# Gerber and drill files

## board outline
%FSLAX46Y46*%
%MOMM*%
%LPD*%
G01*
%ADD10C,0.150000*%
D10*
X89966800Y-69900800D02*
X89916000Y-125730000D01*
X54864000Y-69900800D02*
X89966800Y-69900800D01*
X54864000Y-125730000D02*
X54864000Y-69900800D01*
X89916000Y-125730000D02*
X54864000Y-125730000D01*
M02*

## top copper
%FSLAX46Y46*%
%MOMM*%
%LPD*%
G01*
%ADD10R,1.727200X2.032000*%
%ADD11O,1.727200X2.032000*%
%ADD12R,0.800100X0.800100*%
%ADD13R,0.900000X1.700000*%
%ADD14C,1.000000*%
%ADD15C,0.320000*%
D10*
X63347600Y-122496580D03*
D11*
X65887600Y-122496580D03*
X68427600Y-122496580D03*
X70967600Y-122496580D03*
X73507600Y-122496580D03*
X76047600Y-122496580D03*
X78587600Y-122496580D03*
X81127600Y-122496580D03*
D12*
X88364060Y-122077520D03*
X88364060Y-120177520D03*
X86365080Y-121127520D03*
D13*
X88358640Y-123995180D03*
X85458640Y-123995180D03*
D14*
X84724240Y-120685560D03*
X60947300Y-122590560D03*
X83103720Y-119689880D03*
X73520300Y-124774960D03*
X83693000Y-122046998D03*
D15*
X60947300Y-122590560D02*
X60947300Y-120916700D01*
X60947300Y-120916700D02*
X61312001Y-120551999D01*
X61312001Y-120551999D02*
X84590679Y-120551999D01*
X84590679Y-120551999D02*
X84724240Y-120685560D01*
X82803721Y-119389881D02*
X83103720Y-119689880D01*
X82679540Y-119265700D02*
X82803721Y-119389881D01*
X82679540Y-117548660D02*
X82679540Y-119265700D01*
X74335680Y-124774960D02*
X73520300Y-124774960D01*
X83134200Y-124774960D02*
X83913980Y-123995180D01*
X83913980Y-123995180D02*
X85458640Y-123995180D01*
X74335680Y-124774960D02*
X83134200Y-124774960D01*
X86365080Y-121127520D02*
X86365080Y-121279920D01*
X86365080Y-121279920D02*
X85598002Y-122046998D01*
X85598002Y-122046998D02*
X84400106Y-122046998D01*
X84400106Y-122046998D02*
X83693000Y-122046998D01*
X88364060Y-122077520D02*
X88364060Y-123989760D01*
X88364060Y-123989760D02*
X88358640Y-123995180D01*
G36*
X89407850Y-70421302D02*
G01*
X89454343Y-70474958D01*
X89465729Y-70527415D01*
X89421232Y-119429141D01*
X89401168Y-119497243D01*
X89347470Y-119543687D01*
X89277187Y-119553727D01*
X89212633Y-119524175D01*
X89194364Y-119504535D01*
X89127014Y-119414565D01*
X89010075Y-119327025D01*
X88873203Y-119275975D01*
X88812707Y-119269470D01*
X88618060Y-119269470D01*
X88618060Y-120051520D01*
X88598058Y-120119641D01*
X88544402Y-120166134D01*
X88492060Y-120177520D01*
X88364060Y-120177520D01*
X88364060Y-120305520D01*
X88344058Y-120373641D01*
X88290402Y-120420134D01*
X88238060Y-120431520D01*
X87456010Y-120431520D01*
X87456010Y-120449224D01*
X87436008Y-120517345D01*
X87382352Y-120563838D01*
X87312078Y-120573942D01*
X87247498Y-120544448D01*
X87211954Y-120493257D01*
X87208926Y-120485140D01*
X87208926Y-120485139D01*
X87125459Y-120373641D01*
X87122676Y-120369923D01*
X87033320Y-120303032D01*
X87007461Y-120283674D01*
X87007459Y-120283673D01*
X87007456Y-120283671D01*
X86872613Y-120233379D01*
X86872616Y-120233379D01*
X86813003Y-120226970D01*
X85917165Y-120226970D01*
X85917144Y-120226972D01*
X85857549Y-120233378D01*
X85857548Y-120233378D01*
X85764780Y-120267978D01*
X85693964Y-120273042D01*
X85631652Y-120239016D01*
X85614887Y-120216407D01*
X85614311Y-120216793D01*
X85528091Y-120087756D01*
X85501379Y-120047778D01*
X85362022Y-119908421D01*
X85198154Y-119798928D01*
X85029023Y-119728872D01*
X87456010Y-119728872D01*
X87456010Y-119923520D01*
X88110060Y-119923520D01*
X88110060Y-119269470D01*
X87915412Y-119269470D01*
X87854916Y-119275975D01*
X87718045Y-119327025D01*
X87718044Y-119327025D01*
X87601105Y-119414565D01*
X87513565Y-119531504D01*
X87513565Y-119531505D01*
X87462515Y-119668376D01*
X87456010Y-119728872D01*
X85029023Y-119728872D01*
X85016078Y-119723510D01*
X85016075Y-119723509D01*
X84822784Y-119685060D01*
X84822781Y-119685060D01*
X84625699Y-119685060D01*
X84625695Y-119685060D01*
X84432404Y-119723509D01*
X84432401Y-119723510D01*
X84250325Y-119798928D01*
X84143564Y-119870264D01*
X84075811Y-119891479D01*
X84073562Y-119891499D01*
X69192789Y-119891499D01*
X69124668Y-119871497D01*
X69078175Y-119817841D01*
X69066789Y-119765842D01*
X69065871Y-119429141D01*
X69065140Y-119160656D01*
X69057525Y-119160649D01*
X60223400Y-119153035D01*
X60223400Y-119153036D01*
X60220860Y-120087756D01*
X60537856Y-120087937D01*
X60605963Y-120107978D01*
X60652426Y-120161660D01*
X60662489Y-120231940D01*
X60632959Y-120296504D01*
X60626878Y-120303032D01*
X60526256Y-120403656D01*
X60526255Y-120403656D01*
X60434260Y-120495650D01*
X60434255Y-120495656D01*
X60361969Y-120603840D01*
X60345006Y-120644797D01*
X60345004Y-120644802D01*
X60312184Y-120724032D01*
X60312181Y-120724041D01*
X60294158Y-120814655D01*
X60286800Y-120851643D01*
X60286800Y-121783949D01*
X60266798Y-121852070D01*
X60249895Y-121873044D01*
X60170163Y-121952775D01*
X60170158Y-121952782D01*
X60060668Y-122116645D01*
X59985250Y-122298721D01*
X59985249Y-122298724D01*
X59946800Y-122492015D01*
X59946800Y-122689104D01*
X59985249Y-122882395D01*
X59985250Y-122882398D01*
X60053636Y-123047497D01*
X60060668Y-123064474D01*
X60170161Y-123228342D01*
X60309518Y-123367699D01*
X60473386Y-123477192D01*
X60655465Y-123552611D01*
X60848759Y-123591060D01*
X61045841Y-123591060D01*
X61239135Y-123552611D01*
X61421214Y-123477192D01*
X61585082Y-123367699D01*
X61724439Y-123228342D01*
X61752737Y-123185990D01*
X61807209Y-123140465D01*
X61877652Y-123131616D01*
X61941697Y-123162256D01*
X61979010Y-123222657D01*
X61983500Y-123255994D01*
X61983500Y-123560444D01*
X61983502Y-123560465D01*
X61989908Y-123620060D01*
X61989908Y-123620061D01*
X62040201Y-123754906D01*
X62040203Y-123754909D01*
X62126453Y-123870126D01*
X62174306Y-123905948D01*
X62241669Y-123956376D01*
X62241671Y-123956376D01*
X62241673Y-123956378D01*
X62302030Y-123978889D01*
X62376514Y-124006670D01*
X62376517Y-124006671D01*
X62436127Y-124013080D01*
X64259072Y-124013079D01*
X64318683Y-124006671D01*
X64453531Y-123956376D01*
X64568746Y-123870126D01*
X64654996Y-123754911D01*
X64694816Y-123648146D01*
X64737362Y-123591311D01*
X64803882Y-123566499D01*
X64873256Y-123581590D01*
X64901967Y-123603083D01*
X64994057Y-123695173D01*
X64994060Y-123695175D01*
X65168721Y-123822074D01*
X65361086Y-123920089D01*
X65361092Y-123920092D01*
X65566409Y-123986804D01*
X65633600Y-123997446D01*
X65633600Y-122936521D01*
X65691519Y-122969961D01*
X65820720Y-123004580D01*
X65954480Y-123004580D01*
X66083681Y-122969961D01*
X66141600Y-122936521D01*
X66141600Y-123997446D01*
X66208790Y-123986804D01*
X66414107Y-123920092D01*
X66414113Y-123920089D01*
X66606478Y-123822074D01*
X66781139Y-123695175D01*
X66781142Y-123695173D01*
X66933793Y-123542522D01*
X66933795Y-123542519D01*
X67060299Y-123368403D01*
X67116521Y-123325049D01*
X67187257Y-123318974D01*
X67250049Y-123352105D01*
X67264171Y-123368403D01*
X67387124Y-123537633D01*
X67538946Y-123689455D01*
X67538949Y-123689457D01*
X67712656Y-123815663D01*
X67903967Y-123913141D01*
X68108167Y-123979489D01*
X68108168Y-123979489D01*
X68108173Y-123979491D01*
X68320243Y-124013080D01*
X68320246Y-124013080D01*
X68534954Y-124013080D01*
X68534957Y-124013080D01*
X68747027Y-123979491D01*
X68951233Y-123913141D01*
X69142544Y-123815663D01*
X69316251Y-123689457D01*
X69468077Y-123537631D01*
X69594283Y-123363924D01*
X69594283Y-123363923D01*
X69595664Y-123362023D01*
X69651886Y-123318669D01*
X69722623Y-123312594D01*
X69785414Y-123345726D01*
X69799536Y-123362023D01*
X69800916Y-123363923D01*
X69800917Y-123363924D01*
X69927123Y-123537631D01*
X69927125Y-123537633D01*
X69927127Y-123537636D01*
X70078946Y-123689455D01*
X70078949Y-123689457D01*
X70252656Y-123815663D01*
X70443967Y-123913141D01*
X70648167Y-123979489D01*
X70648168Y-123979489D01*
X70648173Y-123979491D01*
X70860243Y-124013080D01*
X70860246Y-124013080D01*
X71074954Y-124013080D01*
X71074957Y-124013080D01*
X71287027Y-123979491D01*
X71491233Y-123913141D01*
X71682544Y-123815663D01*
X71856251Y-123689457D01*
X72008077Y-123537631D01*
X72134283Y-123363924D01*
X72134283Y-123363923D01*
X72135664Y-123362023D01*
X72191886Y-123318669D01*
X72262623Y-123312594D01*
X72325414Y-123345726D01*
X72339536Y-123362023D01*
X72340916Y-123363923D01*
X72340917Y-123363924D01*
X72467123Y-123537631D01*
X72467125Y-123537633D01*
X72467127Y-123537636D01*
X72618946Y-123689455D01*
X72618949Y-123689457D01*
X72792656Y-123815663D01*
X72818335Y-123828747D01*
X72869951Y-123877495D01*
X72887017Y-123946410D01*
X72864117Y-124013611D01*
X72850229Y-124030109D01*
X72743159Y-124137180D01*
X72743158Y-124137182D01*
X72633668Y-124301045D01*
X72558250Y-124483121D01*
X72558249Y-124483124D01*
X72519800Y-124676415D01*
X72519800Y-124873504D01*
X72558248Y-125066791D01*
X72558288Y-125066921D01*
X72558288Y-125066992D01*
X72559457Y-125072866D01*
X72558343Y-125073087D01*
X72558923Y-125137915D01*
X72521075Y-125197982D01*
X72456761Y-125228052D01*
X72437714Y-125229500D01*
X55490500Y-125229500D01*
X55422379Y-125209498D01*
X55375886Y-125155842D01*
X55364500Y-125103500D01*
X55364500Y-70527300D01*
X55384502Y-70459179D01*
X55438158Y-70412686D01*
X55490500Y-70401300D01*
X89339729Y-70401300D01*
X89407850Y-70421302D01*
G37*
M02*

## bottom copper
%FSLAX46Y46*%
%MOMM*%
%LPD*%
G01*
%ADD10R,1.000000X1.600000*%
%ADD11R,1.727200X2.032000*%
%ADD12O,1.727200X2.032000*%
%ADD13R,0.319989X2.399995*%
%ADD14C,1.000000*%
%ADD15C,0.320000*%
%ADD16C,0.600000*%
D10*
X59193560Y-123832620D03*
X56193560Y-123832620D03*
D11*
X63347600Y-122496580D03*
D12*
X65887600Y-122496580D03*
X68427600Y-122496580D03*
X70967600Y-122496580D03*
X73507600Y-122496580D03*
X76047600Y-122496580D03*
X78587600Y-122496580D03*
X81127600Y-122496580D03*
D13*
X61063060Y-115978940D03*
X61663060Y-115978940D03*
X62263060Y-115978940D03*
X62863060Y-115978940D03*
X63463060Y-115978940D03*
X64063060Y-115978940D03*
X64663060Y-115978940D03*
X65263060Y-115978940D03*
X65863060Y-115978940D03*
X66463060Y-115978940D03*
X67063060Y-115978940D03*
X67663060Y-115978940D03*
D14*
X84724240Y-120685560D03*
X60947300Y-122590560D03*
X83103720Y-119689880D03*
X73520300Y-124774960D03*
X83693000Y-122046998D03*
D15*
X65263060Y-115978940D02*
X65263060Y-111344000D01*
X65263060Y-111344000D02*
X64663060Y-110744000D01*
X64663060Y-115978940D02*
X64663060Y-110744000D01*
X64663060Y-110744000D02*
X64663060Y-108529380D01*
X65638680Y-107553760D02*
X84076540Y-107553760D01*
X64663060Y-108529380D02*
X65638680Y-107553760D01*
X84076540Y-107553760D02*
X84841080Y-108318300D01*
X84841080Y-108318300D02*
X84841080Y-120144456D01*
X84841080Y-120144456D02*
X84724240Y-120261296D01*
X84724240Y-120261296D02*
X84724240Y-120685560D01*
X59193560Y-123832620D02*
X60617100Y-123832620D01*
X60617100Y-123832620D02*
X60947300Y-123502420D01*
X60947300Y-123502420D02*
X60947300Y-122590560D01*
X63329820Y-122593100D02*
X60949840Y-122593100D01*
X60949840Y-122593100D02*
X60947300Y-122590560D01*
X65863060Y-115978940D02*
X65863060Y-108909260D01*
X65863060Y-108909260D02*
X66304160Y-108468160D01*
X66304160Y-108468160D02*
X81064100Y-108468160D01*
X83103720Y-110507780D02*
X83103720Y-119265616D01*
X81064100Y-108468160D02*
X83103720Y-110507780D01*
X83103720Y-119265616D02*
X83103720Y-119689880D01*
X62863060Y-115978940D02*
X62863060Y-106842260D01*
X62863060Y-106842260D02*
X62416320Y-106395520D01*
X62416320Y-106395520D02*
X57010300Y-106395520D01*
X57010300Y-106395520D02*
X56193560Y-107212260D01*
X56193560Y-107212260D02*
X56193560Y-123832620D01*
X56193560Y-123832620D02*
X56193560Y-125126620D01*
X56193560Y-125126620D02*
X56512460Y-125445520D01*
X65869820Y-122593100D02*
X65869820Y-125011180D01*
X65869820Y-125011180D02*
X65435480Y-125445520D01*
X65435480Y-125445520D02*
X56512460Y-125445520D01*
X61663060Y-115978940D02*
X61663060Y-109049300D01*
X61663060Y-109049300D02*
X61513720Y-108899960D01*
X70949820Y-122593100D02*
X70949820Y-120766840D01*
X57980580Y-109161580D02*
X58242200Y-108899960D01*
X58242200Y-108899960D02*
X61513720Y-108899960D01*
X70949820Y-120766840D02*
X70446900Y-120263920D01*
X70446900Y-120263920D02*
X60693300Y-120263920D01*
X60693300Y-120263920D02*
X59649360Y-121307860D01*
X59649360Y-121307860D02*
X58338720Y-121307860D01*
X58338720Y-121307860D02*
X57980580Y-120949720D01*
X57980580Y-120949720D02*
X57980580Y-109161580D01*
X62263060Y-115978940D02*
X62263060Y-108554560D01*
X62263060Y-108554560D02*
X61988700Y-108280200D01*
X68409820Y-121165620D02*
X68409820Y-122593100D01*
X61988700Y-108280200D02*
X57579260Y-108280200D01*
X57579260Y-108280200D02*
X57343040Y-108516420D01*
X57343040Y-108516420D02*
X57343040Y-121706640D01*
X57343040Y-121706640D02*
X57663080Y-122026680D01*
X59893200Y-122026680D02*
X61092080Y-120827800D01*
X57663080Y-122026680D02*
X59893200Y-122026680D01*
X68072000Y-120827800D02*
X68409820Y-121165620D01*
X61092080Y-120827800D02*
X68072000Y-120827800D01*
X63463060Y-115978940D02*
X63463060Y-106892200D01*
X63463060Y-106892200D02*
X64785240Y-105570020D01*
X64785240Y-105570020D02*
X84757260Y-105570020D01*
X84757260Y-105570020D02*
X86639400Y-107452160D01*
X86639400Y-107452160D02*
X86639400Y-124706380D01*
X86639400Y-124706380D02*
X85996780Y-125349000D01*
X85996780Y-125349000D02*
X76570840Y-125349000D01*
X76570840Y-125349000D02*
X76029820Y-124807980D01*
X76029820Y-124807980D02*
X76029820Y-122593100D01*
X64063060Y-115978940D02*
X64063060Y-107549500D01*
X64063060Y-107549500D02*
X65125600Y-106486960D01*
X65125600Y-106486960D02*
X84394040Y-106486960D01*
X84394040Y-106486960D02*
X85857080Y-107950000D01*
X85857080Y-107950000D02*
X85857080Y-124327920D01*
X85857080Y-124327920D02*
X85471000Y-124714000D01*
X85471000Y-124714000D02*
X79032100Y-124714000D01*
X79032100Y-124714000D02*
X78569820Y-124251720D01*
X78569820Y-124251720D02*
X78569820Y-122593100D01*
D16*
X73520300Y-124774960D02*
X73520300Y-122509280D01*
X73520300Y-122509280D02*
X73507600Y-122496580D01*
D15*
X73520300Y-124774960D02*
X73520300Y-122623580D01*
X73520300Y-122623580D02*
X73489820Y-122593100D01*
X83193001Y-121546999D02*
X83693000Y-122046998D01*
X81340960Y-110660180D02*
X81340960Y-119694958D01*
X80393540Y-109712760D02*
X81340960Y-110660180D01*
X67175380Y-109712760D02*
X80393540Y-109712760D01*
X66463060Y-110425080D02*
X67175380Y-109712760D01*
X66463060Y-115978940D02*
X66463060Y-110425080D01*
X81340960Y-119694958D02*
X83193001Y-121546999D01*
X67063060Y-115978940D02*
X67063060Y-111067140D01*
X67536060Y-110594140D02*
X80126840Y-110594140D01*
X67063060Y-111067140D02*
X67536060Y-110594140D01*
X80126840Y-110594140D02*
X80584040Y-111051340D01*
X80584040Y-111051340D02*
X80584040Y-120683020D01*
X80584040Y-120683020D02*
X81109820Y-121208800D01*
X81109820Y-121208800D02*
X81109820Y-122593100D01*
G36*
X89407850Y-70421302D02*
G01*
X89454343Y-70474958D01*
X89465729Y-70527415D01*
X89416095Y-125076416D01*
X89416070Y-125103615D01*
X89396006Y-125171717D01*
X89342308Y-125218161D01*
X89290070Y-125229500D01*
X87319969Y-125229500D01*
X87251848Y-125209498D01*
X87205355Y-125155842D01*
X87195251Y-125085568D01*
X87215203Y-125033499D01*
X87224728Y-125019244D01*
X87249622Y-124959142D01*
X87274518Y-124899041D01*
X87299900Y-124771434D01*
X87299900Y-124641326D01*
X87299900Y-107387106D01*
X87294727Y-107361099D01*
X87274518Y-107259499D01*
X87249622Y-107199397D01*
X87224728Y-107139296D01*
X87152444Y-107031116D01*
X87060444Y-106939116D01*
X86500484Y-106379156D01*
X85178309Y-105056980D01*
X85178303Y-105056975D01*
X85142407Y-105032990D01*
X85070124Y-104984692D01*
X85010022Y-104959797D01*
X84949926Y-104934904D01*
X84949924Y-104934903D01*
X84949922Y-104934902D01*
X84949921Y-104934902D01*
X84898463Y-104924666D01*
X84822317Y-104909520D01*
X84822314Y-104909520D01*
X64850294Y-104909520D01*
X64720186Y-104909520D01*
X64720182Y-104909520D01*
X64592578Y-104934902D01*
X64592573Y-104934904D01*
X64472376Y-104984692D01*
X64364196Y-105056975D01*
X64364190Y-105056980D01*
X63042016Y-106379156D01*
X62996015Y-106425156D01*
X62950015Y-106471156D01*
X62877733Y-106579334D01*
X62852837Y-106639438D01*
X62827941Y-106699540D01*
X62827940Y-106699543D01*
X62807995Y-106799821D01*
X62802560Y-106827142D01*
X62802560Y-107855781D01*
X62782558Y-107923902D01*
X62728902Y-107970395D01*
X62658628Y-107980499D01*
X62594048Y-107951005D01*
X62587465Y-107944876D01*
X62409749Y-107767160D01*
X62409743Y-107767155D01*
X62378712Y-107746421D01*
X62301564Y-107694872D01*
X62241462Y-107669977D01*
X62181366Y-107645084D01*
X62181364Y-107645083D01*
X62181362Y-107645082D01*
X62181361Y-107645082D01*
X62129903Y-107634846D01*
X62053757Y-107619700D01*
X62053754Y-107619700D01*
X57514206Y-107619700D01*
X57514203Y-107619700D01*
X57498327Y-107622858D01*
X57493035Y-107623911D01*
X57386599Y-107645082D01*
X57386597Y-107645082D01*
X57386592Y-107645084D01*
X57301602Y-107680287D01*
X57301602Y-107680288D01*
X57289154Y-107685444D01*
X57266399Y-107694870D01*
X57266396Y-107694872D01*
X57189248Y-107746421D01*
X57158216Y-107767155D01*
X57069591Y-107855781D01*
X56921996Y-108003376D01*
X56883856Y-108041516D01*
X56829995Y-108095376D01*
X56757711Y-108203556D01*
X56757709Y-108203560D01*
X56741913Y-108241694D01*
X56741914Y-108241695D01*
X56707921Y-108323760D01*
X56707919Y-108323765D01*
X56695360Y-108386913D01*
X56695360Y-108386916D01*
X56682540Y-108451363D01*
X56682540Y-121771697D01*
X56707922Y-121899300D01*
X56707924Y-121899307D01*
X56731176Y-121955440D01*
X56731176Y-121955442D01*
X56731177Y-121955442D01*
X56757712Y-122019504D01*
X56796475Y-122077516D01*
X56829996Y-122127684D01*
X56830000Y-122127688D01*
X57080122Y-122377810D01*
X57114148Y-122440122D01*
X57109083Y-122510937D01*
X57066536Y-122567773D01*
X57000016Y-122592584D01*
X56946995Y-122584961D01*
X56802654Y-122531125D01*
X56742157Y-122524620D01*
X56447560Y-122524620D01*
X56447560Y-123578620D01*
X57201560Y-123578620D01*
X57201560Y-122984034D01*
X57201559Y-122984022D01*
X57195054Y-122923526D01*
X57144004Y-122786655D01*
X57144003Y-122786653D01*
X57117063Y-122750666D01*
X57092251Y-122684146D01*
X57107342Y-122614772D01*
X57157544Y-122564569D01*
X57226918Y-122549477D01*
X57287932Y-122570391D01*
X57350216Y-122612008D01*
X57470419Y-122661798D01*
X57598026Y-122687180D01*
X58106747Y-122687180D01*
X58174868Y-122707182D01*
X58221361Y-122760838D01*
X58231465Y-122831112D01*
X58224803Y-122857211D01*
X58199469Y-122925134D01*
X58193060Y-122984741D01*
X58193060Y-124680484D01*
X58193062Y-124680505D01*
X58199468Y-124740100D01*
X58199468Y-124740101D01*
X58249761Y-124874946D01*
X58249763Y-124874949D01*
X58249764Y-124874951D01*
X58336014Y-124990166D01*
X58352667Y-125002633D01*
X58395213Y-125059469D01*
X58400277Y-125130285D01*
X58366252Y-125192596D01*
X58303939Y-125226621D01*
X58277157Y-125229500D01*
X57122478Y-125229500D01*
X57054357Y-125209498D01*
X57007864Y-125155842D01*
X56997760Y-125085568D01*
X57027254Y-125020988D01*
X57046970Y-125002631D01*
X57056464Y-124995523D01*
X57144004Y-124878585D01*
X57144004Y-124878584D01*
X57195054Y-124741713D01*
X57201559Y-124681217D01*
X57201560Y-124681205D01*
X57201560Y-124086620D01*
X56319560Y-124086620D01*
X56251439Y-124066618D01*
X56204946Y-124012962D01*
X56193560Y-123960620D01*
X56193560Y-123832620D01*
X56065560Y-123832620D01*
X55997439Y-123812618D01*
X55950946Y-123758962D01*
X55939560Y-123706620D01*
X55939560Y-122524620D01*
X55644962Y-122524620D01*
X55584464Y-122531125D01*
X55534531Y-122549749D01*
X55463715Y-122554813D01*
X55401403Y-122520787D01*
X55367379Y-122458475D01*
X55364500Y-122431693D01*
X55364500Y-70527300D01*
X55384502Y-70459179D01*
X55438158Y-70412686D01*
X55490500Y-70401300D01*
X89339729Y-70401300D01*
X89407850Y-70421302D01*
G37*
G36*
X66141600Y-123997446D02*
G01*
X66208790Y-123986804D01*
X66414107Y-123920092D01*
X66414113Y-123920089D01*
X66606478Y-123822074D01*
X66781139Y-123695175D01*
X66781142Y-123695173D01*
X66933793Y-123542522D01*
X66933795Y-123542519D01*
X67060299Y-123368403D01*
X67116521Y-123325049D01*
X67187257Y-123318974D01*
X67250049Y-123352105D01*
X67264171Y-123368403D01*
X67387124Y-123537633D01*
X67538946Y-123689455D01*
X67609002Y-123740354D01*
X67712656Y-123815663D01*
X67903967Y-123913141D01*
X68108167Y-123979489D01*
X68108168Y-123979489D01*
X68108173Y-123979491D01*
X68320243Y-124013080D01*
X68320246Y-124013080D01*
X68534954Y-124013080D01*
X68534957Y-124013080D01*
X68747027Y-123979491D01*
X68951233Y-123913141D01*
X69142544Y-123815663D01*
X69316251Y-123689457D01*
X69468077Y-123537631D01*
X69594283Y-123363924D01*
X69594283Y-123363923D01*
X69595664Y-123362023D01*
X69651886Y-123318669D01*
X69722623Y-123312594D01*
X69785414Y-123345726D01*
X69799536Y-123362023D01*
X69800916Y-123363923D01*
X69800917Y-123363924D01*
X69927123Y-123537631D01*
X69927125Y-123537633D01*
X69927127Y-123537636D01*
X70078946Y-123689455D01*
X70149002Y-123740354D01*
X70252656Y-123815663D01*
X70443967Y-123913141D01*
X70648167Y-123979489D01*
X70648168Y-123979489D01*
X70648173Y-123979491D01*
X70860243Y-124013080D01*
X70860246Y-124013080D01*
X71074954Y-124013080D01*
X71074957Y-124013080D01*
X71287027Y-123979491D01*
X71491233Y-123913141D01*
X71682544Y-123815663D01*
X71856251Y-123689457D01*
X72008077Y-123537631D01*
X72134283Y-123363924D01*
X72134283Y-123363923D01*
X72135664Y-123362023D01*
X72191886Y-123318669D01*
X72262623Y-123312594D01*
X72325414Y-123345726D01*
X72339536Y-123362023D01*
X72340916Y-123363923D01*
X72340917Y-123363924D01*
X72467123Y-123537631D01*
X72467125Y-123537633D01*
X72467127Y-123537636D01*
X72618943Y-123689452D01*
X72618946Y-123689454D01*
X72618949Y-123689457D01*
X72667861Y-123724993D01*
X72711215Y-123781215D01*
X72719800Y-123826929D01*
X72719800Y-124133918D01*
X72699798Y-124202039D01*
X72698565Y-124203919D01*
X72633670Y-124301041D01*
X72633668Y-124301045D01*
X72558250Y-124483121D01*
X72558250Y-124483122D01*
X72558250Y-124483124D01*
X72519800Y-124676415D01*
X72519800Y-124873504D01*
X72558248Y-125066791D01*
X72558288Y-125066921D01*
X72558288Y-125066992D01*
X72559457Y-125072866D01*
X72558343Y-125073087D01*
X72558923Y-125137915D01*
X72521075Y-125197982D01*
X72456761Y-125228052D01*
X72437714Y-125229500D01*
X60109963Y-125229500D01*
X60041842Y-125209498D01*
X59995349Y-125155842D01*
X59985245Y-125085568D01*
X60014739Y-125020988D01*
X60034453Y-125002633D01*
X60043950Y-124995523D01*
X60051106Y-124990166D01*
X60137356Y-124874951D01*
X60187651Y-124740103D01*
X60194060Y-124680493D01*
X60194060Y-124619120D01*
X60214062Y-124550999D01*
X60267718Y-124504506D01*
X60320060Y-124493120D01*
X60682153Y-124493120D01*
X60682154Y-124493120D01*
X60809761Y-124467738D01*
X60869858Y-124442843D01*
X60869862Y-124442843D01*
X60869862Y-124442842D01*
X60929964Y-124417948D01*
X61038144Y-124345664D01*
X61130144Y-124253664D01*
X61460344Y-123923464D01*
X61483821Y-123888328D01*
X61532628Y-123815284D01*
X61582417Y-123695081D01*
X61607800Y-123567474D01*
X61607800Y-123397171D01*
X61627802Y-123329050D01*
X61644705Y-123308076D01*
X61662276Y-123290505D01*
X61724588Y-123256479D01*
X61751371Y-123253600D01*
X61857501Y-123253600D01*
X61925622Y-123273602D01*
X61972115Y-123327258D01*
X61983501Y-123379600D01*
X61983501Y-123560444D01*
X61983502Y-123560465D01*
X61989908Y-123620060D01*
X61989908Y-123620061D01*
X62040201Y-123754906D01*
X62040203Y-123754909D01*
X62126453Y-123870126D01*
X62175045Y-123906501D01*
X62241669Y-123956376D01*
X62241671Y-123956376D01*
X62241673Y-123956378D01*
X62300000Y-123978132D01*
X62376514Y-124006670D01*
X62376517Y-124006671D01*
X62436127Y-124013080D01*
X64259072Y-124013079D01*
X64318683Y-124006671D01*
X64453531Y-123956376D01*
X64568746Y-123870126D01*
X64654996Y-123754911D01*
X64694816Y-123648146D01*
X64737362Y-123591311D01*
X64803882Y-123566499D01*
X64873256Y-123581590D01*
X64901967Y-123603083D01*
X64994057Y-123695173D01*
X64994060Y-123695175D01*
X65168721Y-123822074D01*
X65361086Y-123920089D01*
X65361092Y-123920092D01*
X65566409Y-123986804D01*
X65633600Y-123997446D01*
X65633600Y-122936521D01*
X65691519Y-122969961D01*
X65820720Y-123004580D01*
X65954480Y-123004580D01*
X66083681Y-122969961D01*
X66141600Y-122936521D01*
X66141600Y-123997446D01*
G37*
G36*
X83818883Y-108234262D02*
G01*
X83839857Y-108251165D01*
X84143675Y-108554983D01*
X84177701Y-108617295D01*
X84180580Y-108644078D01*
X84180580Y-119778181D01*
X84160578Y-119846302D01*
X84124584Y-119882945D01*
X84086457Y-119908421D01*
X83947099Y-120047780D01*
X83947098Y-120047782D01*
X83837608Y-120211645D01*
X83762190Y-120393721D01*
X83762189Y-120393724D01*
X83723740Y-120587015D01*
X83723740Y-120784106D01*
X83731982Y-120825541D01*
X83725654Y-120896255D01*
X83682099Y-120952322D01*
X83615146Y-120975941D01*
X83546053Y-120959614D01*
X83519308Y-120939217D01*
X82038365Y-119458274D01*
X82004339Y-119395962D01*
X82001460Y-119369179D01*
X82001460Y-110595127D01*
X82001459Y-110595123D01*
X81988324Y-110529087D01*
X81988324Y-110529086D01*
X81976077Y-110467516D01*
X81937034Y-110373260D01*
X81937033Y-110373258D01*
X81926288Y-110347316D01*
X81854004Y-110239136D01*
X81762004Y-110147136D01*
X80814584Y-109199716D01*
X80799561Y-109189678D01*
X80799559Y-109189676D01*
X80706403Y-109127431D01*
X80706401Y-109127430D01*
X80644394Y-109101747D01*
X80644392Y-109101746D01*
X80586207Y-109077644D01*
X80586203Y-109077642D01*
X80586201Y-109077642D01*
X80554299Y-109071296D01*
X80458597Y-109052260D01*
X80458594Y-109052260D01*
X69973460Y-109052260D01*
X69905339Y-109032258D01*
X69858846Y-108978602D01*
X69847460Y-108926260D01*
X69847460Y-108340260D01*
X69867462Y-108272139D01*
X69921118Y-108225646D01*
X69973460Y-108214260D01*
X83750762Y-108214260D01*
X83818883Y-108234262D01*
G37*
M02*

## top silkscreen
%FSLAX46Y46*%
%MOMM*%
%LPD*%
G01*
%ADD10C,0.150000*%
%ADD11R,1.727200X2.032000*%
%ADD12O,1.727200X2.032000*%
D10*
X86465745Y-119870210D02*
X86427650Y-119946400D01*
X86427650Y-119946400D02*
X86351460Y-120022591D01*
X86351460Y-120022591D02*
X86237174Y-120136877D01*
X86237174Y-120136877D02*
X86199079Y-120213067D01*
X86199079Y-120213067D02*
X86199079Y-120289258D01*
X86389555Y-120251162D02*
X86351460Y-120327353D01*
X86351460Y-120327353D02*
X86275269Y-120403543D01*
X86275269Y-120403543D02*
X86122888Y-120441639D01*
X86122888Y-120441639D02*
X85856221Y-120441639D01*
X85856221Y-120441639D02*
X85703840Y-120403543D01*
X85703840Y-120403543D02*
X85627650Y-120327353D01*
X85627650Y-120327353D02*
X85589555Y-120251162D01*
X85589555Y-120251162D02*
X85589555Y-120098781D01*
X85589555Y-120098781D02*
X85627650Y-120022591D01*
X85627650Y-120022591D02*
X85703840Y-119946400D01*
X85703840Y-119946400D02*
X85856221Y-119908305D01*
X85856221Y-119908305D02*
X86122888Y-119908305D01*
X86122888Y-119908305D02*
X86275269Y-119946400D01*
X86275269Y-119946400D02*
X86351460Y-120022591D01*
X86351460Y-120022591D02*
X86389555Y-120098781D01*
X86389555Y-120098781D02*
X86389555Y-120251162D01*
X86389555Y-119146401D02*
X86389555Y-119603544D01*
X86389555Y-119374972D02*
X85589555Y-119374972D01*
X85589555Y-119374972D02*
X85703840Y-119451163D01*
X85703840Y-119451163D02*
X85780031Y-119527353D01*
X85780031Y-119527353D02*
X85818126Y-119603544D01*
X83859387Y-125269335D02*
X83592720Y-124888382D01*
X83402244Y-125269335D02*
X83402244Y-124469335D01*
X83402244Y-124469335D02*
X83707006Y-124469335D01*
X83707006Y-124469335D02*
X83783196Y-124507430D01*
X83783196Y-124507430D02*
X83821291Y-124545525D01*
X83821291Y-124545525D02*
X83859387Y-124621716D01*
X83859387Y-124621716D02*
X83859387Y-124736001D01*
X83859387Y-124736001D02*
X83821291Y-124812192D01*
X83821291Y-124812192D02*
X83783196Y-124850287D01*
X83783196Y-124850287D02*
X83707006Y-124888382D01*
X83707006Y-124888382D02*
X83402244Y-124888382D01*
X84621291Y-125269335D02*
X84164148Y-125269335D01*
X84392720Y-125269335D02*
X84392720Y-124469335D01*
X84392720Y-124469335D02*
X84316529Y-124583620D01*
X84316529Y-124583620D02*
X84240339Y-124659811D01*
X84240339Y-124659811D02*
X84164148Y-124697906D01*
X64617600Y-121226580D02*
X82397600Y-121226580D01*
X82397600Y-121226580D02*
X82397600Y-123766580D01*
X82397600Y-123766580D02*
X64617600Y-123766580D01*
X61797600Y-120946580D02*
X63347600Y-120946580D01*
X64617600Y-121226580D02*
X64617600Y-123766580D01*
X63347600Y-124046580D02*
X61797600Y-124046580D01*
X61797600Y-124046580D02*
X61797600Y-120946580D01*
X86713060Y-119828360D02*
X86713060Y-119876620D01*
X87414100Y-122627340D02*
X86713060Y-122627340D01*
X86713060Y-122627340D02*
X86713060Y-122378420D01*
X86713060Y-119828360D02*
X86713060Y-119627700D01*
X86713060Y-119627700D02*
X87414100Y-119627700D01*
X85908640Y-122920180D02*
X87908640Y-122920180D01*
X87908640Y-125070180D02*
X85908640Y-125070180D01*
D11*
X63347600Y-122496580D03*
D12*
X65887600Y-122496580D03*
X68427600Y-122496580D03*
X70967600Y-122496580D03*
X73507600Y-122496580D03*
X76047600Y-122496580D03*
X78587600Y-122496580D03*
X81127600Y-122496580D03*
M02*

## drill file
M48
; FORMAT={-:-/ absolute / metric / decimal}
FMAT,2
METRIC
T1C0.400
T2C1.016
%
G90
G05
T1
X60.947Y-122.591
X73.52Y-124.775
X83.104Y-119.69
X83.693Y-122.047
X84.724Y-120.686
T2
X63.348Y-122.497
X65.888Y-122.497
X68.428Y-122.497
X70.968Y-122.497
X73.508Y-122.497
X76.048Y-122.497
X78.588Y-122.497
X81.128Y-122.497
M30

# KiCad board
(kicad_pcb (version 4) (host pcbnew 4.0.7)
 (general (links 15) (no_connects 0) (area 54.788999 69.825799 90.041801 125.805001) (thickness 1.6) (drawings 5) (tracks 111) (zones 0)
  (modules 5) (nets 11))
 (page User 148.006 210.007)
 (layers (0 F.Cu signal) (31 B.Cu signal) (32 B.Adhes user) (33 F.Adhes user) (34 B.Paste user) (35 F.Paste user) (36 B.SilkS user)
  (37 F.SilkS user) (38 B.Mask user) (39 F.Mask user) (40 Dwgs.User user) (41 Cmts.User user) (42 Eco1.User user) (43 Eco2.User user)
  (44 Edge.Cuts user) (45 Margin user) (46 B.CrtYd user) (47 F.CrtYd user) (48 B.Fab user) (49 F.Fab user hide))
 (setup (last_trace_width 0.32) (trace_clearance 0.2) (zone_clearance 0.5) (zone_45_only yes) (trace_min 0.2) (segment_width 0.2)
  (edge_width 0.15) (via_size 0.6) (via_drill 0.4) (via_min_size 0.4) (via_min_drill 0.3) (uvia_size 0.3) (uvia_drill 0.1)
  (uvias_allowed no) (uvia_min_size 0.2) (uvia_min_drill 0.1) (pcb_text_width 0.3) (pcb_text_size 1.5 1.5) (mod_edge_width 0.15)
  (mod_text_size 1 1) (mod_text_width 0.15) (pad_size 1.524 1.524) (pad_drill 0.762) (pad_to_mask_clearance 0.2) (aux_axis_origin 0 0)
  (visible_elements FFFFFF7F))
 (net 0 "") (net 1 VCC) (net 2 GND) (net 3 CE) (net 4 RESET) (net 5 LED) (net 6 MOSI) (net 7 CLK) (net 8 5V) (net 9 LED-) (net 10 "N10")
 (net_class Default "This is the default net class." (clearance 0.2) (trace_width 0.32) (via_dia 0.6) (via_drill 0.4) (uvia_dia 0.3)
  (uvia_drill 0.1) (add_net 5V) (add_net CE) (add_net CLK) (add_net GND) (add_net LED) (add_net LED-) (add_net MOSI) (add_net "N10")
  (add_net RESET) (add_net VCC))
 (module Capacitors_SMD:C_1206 (layer B.Cu) (at 57.69356 123.83262 180)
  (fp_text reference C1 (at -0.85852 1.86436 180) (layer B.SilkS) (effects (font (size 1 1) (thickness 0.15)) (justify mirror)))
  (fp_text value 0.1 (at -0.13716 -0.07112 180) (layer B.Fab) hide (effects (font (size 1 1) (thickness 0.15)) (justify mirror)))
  (pad 1 smd rect (at -1.5 0 180) (size 1 1.6) (layers B.Cu B.Paste B.Mask) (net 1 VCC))
  (pad 2 smd rect (at 1.5 0 180) (size 1 1.6) (layers B.Cu B.Paste B.Mask) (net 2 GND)))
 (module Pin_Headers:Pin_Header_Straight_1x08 (layer F.Cu) (at 63.3476 122.49658 90)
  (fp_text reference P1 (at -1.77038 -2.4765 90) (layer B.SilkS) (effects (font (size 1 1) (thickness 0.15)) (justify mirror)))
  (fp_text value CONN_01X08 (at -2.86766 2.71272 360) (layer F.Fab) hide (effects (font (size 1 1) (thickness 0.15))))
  (fp_line (start 1.27 1.27) (end 1.27 19.05) (layer F.SilkS) (width 0.15))
  (fp_line (start 1.27 19.05) (end -1.27 19.05) (layer F.SilkS) (width 0.15))
  (fp_line (start -1.27 19.05) (end -1.27 1.27) (layer F.SilkS) (width 0.15))
  (fp_line (start 1.55 -1.55) (end 1.55 0) (layer F.SilkS) (width 0.15))
  (fp_line (start 1.27 1.27) (end -1.27 1.27) (layer F.SilkS) (width 0.15))
  (fp_line (start -1.55 0) (end -1.55 -1.55) (layer F.SilkS) (width 0.15))
  (fp_line (start -1.55 -1.55) (end 1.55 -1.55) (layer F.SilkS) (width 0.15))
  (pad 1 thru_hole rect (at 0 0 90) (size 2.032 1.7272) (drill 1.016) (layers *.Cu *.Mask F.SilkS) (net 1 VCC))
  (pad 2 thru_hole oval (at 0 2.54 90) (size 2.032 1.7272) (drill 1.016) (layers *.Cu *.Mask F.SilkS) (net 2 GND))
  (pad 3 thru_hole oval (at 0 5.08 90) (size 2.032 1.7272) (drill 1.016) (layers *.Cu *.Mask F.SilkS) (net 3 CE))
  (pad 4 thru_hole oval (at 0 7.62 90) (size 2.032 1.7272) (drill 1.016) (layers *.Cu *.Mask F.SilkS) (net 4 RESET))
  (pad 5 thru_hole oval (at 0 10.16 90) (size 2.032 1.7272) (drill 1.016) (layers *.Cu *.Mask F.SilkS) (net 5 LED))
  (pad 6 thru_hole oval (at 0 12.7 90) (size 2.032 1.7272) (drill 1.016) (layers *.Cu *.Mask F.SilkS) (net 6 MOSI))
  (pad 7 thru_hole oval (at 0 15.24 90) (size 2.032 1.7272) (drill 1.016) (layers *.Cu *.Mask F.SilkS) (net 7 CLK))
  (pad 8 thru_hole oval (at 0 17.78 90) (size 2.032 1.7272) (drill 1.016) (layers *.Cu *.Mask F.SilkS) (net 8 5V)))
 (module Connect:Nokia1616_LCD (layer B.Cu) (at 68.14454 114.77752)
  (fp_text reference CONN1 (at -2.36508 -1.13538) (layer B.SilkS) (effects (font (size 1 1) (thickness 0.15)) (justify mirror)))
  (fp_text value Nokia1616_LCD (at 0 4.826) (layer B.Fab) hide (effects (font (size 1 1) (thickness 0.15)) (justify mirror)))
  (pad 1 smd rect (at -7.08148 1.20142) (size 0.319989 2.399995) (layers B.Cu B.Paste B.Mask))
  (pad 2 smd rect (at -6.48148 1.20142) (size 0.319989 2.399995) (layers B.Cu B.Paste B.Mask) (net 4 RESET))
  (pad 3 smd rect (at -5.88148 1.20142) (size 0.319989 2.399995) (layers B.Cu B.Paste B.Mask) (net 3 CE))
  (pad 4 smd rect (at -5.28148 1.20142) (size 0.319989 2.399995) (layers B.Cu B.Paste B.Mask) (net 2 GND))
  (pad 5 smd rect (at -4.68148 1.20142) (size 0.319989 2.399995) (layers B.Cu B.Paste B.Mask) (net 6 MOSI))
  (pad 6 smd rect (at -4.08148 1.20142) (size 0.319989 2.399995) (layers B.Cu B.Paste B.Mask) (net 7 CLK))
  (pad 7 smd rect (at -3.48148 1.20142) (size 0.319989 2.399995) (layers B.Cu B.Paste B.Mask) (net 1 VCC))
  (pad 8 smd rect (at -2.88148 1.20142) (size 0.319989 2.399995) (layers B.Cu B.Paste B.Mask) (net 1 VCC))
  (pad 9 smd rect (at -2.28148 1.20142) (size 0.319989 2.399995) (layers B.Cu B.Paste B.Mask) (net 2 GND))
  (pad 10 smd rect (at -1.68148 1.20142) (size 0.319989 2.399995) (layers B.Cu B.Paste B.Mask) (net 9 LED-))
  (pad 11 smd rect (at -1.08148 1.20142) (size 0.319989 2.399995) (layers B.Cu B.Paste B.Mask) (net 8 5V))
  (pad 12 smd rect (at -0.48148 1.20142) (size 0.319989 2.399995) (layers B.Cu B.Paste B.Mask)))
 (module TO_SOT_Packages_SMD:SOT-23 (layer F.Cu) (at 87.3633 121.12752 90)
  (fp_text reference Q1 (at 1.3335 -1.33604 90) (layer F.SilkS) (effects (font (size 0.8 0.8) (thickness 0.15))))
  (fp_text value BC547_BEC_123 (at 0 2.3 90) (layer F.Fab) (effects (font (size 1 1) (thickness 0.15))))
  (fp_line (start 1.29916 -0.65024) (end 1.2509 -0.65024) (layer F.SilkS) (width 0.15))
  (fp_line (start -1.49982 0.0508) (end -1.49982 -0.65024) (layer F.SilkS) (width 0.15))
  (fp_line (start -1.49982 -0.65024) (end -1.2509 -0.65024) (layer F.SilkS) (width 0.15))
  (fp_line (start 1.29916 -0.65024) (end 1.49982 -0.65024) (layer F.SilkS) (width 0.15))
  (fp_line (start 1.49982 -0.65024) (end 1.49982 0.0508) (layer F.SilkS) (width 0.15))
  (pad 1 smd rect (at -0.95 1.00076 90) (size 0.8001 0.8001) (layers F.Cu F.Paste F.Mask) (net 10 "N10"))
  (pad 2 smd rect (at 0.95 1.00076 90) (size 0.8001 0.8001) (layers F.Cu F.Paste F.Mask) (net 2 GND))
  (pad 3 smd rect (at 0 -0.99822 90) (size 0.8001 0.8001) (layers F.Cu F.Paste F.Mask) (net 9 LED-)))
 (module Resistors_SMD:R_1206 (layer F.Cu) (at 86.90864 123.99518 180)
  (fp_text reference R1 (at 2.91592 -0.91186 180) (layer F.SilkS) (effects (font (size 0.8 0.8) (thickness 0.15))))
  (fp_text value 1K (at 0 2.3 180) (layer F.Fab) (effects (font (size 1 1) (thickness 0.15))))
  (fp_line (start 1 1.075) (end -1 1.075) (layer F.SilkS) (width 0.15))
  (fp_line (start -1 -1.075) (end 1 -1.075) (layer F.SilkS) (width 0.15))
  (pad 1 smd rect (at -1.45 0 180) (size 0.9 1.7) (layers F.Cu F.Paste F.Mask) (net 10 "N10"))
  (pad 2 smd rect (at 1.45 0 180) (size 0.9 1.7) (layers F.Cu F.Paste F.Mask) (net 5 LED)))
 (gr_line (start 89.9668 69.9008) (end 89.916 125.73) (layer Edge.Cuts) (width 0.15))
 (gr_line (start 54.864 69.9008) (end 89.9668 69.9008) (layer Edge.Cuts) (width 0.15))
 (gr_line (start 54.864 125.73) (end 54.864 69.9008) (layer Edge.Cuts) (width 0.15))
 (gr_line (start 89.916 125.73) (end 54.864 125.73) (layer Edge.Cuts) (width 0.15))
 (segment (start 60.9473 122.59056) (end 60.9473 120.9167) (width 0.32) (layer F.Cu) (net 1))
 (segment (start 60.9473 120.9167) (end 61.312001 120.551999) (width 0.32) (layer F.Cu) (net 1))
 (segment (start 61.312001 120.551999) (end 84.590679 120.551999) (width 0.32) (layer F.Cu) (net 1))
 (segment (start 84.590679 120.551999) (end 84.72424 120.68556) (width 0.32) (layer F.Cu) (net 1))
 (segment (start 65.26306 115.97894) (end 65.26306 111.344) (width 0.32) (layer B.Cu) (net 1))
 (segment (start 65.26306 111.344) (end 64.66306 110.744) (width 0.32) (layer B.Cu) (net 1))
 (segment (start 64.66306 115.97894) (end 64.66306 110.744) (width 0.32) (layer B.Cu) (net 1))
 (segment (start 64.66306 110.744) (end 64.66306 108.52938) (width 0.32) (layer B.Cu) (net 1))
 (segment (start 65.63868 107.55376) (end 84.07654 107.55376) (width 0.32) (layer B.Cu) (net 1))
 (segment (start 64.66306 108.52938) (end 65.63868 107.55376) (width 0.32) (layer B.Cu) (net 1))
 (segment (start 84.07654 107.55376) (end 84.84108 108.3183) (width 0.32) (layer B.Cu) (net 1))
 (segment (start 84.84108 108.3183) (end 84.84108 120.144456) (width 0.32) (layer B.Cu) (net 1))
 (segment (start 84.84108 120.144456) (end 84.72424 120.261296) (width 0.32) (layer B.Cu) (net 1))
 (segment (start 84.72424 120.261296) (end 84.72424 120.68556) (width 0.32) (layer B.Cu) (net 1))
 (segment (start 59.19356 123.83262) (end 60.6171 123.83262) (width 0.32) (layer B.Cu) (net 1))
 (segment (start 60.6171 123.83262) (end 60.9473 123.50242) (width 0.32) (layer B.Cu) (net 1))
 (segment (start 60.9473 123.50242) (end 60.9473 122.59056) (width 0.32) (layer B.Cu) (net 1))
 (via (at 84.72424 120.68556) (size 1) (drill 0.4) (layers F.Cu B.Cu) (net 1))
 (segment (start 63.32982 122.5931) (end 60.94984 122.5931) (width 0.32) (layer B.Cu) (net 1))
 (segment (start 60.94984 122.5931) (end 60.9473 122.59056) (width 0.32) (layer B.Cu) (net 1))
 (via (at 60.9473 122.59056) (size 1) (drill 0.4) (layers F.Cu B.Cu) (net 1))
 (segment (start 65.86306 115.97894) (end 65.86306 108.90926) (width 0.32) (layer B.Cu) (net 2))
 (segment (start 65.86306 108.90926) (end 66.30416 108.46816) (width 0.32) (layer B.Cu) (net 2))
 (segment (start 66.30416 108.46816) (end 81.0641 108.46816) (width 0.32) (layer B.Cu) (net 2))
 (segment (start 83.10372 110.50778) (end 83.10372 119.265616) (width 0.32) (layer B.Cu) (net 2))
 (segment (start 81.0641 108.46816) (end 83.10372 110.50778) (width 0.32) (layer B.Cu) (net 2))
 (segment (start 83.10372 119.265616) (end 83.10372 119.68988) (width 0.32) (layer B.Cu) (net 2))
 (segment (start 62.86306 115.97894) (end 62.86306 106.84226) (width 0.32) (layer B.Cu) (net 2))
 (segment (start 62.86306 106.84226) (end 62.41632 106.39552) (width 0.32) (layer B.Cu) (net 2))
 (segment (start 62.41632 106.39552) (end 57.0103 106.39552) (width 0.32) (layer B.Cu) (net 2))
 (segment (start 57.0103 106.39552) (end 56.19356 107.21226) (width 0.32) (layer B.Cu) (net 2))
 (segment (start 56.19356 107.21226) (end 56.19356 123.83262) (width 0.32) (layer B.Cu) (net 2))
 (segment (start 56.19356 123.83262) (end 56.19356 125.12662) (width 0.32) (layer B.Cu) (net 2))
 (segment (start 56.19356 125.12662) (end 56.51246 125.44552) (width 0.32) (layer B.Cu) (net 2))
 (segment (start 65.86982 122.5931) (end 65.86982 125.01118) (width 0.32) (layer B.Cu) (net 2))
 (segment (start 65.86982 125.01118) (end 65.43548 125.44552) (width 0.32) (layer B.Cu) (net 2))
 (segment (start 65.43548 125.44552) (end 56.51246 125.44552) (width 0.32) (layer B.Cu) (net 2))
 (segment (start 82.803721 119.389881) (end 83.10372 119.68988) (width 0.32) (layer F.Cu) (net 2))
 (segment (start 82.67954 119.2657) (end 82.803721 119.389881) (width 0.32) (layer F.Cu) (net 2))
 (segment (start 82.67954 117.54866) (end 82.67954 119.2657) (width 0.32) (layer F.Cu) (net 2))
 (via (at 83.10372 119.68988) (size 1) (drill 0.4) (layers F.Cu B.Cu) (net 2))
 (segment (start 61.66306 115.97894) (end 61.66306 109.0493) (width 0.32) (layer B.Cu) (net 4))
 (segment (start 61.66306 109.0493) (end 61.51372 108.89996) (width 0.32) (layer B.Cu) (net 4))
 (segment (start 70.94982 122.5931) (end 70.94982 120.76684) (width 0.32) (layer B.Cu) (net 4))
 (segment (start 57.98058 109.16158) (end 58.2422 108.89996) (width 0.32) (layer B.Cu) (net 4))
 (segment (start 58.2422 108.89996) (end 61.51372 108.89996) (width 0.32) (layer B.Cu) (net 4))
 (segment (start 70.94982 120.76684) (end 70.4469 120.26392) (width 0.32) (layer B.Cu) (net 4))
 (segment (start 70.4469 120.26392) (end 60.6933 120.26392) (width 0.32) (layer B.Cu) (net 4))
 (segment (start 60.6933 120.26392) (end 59.64936 121.30786) (width 0.32) (layer B.Cu) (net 4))
 (segment (start 59.64936 121.30786) (end 58.33872 121.30786) (width 0.32) (layer B.Cu) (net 4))
 (segment (start 58.33872 121.30786) (end 57.98058 120.94972) (width 0.32) (layer B.Cu) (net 4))
 (segment (start 57.98058 120.94972) (end 57.98058 109.16158) (width 0.32) (layer B.Cu) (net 4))
 (segment (start 62.26306 115.97894) (end 62.26306 108.55456) (width 0.32) (layer B.Cu) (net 3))
 (segment (start 62.26306 108.55456) (end 61.9887 108.2802) (width 0.32) (layer B.Cu) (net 3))
 (segment (start 68.40982 121.16562) (end 68.40982 122.5931) (width 0.32) (layer B.Cu) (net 3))
 (segment (start 61.9887 108.2802) (end 57.57926 108.2802) (width 0.32) (layer B.Cu) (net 3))
 (segment (start 57.57926 108.2802) (end 57.34304 108.51642) (width 0.32) (layer B.Cu) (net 3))
 (segment (start 57.34304 108.51642) (end 57.34304 121.70664) (width 0.32) (layer B.Cu) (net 3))
 (segment (start 57.34304 121.70664) (end 57.66308 122.02668) (width 0.32) (layer B.Cu) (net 3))
 (segment (start 59.8932 122.02668) (end 61.09208 120.8278) (width 0.32) (layer B.Cu) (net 3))
 (segment (start 57.66308 122.02668) (end 59.8932 122.02668) (width 0.32) (layer B.Cu) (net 3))
 (segment (start 68.072 120.8278) (end 68.40982 121.16562) (width 0.32) (layer B.Cu) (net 3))
 (segment (start 61.09208 120.8278) (end 68.072 120.8278) (width 0.32) (layer B.Cu) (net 3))
 (segment (start 63.46306 115.97894) (end 63.46306 106.8922) (width 0.32) (layer B.Cu) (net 6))
 (segment (start 63.46306 106.8922) (end 64.78524 105.57002) (width 0.32) (layer B.Cu) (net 6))
 (segment (start 64.78524 105.57002) (end 84.75726 105.57002) (width 0.32) (layer B.Cu) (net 6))
 (segment (start 84.75726 105.57002) (end 86.6394 107.45216) (width 0.32) (layer B.Cu) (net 6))
 (segment (start 86.6394 107.45216) (end 86.6394 124.70638) (width 0.32) (layer B.Cu) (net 6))
 (segment (start 86.6394 124.70638) (end 85.99678 125.349) (width 0.32) (layer B.Cu) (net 6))
 (segment (start 85.99678 125.349) (end 76.57084 125.349) (width 0.32) (layer B.Cu) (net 6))
 (segment (start 76.57084 125.349) (end 76.02982 124.80798) (width 0.32) (layer B.Cu) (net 6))
 (segment (start 76.02982 124.80798) (end 76.02982 122.5931) (width 0.32) (layer B.Cu) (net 6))
 (segment (start 64.06306 115.97894) (end 64.06306 107.5495) (width 0.32) (layer B.Cu) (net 7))
 (segment (start 64.06306 107.5495) (end 65.1256 106.48696) (width 0.32) (layer B.Cu) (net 7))
 (segment (start 65.1256 106.48696) (end 84.39404 106.48696) (width 0.32) (layer B.Cu) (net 7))
 (segment (start 84.39404 106.48696) (end 85.85708 107.95) (width 0.32) (layer B.Cu) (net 7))
 (segment (start 85.85708 107.95) (end 85.85708 124.32792) (width 0.32) (layer B.Cu) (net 7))
 (segment (start 85.85708 124.32792) (end 85.471 124.714) (width 0.32) (layer B.Cu) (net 7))
 (segment (start 85.471 124.714) (end 79.0321 124.714) (width 0.32) (layer B.Cu) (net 7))
 (segment (start 79.0321 124.714) (end 78.56982 124.25172) (width 0.32) (layer B.Cu) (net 7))
 (segment (start 78.56982 124.25172) (end 78.56982 122.5931) (width 0.32) (layer B.Cu) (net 7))
 (segment (start 73.5203 124.77496) (end 73.5203 122.50928) (width 0.6) (layer B.Cu) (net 5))
 (segment (start 73.5203 122.50928) (end 73.5076 122.49658) (width 0.6) (layer B.Cu) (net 5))
 (segment (start 73.5203 124.77496) (end 73.5203 122.62358) (width 0.32) (layer B.Cu) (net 5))
 (segment (start 73.5203 122.62358) (end 73.48982 122.5931) (width 0.32) (layer B.Cu) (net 5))
 (segment (start 74.33568 124.77496) (end 73.5203 124.77496) (width 0.32) (layer F.Cu) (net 5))
 (via (at 73.5203 124.77496) (size 1) (drill 0.4) (layers F.Cu B.Cu) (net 5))
 (segment (start 83.1342 124.77496) (end 83.91398 123.99518) (width 0.32) (layer F.Cu) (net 5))
 (segment (start 83.91398 123.99518) (end 85.45864 123.99518) (width 0.32) (layer F.Cu) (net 5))
 (segment (start 74.33568 124.77496) (end 83.1342 124.77496) (width 0.32) (layer F.Cu) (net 5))
 (segment (start 86.36508 121.12752) (end 86.36508 121.27992) (width 0.32) (layer F.Cu) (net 9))
 (segment (start 86.36508 121.27992) (end 85.598002 122.046998) (width 0.32) (layer F.Cu) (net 9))
 (segment (start 85.598002 122.046998) (end 84.400106 122.046998) (width 0.32) (layer F.Cu) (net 9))
 (segment (start 84.400106 122.046998) (end 83.693 122.046998) (width 0.32) (layer F.Cu) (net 9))
 (segment (start 83.193001 121.546999) (end 83.693 122.046998) (width 0.32) (layer B.Cu) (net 9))
 (segment (start 81.34096 110.66018) (end 81.34096 119.694958) (width 0.32) (layer B.Cu) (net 9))
 (segment (start 80.39354 109.71276) (end 81.34096 110.66018) (width 0.32) (layer B.Cu) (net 9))
 (segment (start 67.17538 109.71276) (end 80.39354 109.71276) (width 0.32) (layer B.Cu) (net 9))
 (segment (start 66.46306 110.42508) (end 67.17538 109.71276) (width 0.32) (layer B.Cu) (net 9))
 (segment (start 66.46306 115.97894) (end 66.46306 110.42508) (width 0.32) (layer B.Cu) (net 9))
 (segment (start 81.34096 119.694958) (end 83.193001 121.546999) (width 0.32) (layer B.Cu) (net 9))
 (via (at 83.693 122.046998) (size 1) (drill 0.4) (layers F.Cu B.Cu) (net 9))
 (segment (start 88.36406 122.07752) (end 88.36406 123.98976) (width 0.32) (layer F.Cu) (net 10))
 (segment (start 88.36406 123.98976) (end 88.35864 123.99518) (width 0.32) (layer F.Cu) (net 10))
 (segment (start 67.06306 115.97894) (end 67.06306 111.06714) (width 0.32) (layer B.Cu) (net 8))
 (segment (start 67.53606 110.59414) (end 80.12684 110.59414) (width 0.32) (layer B.Cu) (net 8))
 (segment (start 67.06306 111.06714) (end 67.53606 110.59414) (width 0.32) (layer B.Cu) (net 8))
 (segment (start 80.12684 110.59414) (end 80.58404 111.05134) (width 0.32) (layer B.Cu) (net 8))
 (segment (start 80.58404 111.05134) (end 80.58404 120.68302) (width 0.32) (layer B.Cu) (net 8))
 (segment (start 80.58404 120.68302) (end 81.10982 121.2088) (width 0.32) (layer B.Cu) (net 8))
 (segment (start 81.10982 121.2088) (end 81.10982 122.5931) (width 0.32) (layer B.Cu) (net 8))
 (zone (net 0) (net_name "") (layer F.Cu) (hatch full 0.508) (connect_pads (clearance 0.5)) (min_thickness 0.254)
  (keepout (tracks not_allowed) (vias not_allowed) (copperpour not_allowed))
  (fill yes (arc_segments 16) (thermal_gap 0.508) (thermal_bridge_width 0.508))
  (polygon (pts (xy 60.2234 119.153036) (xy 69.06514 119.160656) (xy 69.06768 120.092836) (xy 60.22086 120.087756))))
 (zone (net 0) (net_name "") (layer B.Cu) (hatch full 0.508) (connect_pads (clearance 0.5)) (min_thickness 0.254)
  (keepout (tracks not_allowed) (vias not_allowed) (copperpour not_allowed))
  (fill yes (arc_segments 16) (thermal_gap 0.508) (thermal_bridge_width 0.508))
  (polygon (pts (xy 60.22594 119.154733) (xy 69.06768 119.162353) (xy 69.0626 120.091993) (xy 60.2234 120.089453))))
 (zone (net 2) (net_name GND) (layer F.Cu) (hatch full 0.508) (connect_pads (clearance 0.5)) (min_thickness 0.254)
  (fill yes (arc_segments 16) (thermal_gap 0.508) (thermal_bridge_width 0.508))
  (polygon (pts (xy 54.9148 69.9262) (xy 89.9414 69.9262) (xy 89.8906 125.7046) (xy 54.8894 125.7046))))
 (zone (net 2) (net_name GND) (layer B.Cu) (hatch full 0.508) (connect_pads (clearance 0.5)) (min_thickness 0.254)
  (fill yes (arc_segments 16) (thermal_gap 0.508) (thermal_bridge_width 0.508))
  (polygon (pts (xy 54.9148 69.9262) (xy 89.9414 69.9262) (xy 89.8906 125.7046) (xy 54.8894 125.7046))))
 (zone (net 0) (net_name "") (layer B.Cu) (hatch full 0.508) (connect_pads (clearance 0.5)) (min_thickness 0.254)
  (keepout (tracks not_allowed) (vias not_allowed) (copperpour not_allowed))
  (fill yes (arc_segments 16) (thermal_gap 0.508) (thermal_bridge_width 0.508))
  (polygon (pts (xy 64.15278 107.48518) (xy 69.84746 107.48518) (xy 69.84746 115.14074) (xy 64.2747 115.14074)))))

